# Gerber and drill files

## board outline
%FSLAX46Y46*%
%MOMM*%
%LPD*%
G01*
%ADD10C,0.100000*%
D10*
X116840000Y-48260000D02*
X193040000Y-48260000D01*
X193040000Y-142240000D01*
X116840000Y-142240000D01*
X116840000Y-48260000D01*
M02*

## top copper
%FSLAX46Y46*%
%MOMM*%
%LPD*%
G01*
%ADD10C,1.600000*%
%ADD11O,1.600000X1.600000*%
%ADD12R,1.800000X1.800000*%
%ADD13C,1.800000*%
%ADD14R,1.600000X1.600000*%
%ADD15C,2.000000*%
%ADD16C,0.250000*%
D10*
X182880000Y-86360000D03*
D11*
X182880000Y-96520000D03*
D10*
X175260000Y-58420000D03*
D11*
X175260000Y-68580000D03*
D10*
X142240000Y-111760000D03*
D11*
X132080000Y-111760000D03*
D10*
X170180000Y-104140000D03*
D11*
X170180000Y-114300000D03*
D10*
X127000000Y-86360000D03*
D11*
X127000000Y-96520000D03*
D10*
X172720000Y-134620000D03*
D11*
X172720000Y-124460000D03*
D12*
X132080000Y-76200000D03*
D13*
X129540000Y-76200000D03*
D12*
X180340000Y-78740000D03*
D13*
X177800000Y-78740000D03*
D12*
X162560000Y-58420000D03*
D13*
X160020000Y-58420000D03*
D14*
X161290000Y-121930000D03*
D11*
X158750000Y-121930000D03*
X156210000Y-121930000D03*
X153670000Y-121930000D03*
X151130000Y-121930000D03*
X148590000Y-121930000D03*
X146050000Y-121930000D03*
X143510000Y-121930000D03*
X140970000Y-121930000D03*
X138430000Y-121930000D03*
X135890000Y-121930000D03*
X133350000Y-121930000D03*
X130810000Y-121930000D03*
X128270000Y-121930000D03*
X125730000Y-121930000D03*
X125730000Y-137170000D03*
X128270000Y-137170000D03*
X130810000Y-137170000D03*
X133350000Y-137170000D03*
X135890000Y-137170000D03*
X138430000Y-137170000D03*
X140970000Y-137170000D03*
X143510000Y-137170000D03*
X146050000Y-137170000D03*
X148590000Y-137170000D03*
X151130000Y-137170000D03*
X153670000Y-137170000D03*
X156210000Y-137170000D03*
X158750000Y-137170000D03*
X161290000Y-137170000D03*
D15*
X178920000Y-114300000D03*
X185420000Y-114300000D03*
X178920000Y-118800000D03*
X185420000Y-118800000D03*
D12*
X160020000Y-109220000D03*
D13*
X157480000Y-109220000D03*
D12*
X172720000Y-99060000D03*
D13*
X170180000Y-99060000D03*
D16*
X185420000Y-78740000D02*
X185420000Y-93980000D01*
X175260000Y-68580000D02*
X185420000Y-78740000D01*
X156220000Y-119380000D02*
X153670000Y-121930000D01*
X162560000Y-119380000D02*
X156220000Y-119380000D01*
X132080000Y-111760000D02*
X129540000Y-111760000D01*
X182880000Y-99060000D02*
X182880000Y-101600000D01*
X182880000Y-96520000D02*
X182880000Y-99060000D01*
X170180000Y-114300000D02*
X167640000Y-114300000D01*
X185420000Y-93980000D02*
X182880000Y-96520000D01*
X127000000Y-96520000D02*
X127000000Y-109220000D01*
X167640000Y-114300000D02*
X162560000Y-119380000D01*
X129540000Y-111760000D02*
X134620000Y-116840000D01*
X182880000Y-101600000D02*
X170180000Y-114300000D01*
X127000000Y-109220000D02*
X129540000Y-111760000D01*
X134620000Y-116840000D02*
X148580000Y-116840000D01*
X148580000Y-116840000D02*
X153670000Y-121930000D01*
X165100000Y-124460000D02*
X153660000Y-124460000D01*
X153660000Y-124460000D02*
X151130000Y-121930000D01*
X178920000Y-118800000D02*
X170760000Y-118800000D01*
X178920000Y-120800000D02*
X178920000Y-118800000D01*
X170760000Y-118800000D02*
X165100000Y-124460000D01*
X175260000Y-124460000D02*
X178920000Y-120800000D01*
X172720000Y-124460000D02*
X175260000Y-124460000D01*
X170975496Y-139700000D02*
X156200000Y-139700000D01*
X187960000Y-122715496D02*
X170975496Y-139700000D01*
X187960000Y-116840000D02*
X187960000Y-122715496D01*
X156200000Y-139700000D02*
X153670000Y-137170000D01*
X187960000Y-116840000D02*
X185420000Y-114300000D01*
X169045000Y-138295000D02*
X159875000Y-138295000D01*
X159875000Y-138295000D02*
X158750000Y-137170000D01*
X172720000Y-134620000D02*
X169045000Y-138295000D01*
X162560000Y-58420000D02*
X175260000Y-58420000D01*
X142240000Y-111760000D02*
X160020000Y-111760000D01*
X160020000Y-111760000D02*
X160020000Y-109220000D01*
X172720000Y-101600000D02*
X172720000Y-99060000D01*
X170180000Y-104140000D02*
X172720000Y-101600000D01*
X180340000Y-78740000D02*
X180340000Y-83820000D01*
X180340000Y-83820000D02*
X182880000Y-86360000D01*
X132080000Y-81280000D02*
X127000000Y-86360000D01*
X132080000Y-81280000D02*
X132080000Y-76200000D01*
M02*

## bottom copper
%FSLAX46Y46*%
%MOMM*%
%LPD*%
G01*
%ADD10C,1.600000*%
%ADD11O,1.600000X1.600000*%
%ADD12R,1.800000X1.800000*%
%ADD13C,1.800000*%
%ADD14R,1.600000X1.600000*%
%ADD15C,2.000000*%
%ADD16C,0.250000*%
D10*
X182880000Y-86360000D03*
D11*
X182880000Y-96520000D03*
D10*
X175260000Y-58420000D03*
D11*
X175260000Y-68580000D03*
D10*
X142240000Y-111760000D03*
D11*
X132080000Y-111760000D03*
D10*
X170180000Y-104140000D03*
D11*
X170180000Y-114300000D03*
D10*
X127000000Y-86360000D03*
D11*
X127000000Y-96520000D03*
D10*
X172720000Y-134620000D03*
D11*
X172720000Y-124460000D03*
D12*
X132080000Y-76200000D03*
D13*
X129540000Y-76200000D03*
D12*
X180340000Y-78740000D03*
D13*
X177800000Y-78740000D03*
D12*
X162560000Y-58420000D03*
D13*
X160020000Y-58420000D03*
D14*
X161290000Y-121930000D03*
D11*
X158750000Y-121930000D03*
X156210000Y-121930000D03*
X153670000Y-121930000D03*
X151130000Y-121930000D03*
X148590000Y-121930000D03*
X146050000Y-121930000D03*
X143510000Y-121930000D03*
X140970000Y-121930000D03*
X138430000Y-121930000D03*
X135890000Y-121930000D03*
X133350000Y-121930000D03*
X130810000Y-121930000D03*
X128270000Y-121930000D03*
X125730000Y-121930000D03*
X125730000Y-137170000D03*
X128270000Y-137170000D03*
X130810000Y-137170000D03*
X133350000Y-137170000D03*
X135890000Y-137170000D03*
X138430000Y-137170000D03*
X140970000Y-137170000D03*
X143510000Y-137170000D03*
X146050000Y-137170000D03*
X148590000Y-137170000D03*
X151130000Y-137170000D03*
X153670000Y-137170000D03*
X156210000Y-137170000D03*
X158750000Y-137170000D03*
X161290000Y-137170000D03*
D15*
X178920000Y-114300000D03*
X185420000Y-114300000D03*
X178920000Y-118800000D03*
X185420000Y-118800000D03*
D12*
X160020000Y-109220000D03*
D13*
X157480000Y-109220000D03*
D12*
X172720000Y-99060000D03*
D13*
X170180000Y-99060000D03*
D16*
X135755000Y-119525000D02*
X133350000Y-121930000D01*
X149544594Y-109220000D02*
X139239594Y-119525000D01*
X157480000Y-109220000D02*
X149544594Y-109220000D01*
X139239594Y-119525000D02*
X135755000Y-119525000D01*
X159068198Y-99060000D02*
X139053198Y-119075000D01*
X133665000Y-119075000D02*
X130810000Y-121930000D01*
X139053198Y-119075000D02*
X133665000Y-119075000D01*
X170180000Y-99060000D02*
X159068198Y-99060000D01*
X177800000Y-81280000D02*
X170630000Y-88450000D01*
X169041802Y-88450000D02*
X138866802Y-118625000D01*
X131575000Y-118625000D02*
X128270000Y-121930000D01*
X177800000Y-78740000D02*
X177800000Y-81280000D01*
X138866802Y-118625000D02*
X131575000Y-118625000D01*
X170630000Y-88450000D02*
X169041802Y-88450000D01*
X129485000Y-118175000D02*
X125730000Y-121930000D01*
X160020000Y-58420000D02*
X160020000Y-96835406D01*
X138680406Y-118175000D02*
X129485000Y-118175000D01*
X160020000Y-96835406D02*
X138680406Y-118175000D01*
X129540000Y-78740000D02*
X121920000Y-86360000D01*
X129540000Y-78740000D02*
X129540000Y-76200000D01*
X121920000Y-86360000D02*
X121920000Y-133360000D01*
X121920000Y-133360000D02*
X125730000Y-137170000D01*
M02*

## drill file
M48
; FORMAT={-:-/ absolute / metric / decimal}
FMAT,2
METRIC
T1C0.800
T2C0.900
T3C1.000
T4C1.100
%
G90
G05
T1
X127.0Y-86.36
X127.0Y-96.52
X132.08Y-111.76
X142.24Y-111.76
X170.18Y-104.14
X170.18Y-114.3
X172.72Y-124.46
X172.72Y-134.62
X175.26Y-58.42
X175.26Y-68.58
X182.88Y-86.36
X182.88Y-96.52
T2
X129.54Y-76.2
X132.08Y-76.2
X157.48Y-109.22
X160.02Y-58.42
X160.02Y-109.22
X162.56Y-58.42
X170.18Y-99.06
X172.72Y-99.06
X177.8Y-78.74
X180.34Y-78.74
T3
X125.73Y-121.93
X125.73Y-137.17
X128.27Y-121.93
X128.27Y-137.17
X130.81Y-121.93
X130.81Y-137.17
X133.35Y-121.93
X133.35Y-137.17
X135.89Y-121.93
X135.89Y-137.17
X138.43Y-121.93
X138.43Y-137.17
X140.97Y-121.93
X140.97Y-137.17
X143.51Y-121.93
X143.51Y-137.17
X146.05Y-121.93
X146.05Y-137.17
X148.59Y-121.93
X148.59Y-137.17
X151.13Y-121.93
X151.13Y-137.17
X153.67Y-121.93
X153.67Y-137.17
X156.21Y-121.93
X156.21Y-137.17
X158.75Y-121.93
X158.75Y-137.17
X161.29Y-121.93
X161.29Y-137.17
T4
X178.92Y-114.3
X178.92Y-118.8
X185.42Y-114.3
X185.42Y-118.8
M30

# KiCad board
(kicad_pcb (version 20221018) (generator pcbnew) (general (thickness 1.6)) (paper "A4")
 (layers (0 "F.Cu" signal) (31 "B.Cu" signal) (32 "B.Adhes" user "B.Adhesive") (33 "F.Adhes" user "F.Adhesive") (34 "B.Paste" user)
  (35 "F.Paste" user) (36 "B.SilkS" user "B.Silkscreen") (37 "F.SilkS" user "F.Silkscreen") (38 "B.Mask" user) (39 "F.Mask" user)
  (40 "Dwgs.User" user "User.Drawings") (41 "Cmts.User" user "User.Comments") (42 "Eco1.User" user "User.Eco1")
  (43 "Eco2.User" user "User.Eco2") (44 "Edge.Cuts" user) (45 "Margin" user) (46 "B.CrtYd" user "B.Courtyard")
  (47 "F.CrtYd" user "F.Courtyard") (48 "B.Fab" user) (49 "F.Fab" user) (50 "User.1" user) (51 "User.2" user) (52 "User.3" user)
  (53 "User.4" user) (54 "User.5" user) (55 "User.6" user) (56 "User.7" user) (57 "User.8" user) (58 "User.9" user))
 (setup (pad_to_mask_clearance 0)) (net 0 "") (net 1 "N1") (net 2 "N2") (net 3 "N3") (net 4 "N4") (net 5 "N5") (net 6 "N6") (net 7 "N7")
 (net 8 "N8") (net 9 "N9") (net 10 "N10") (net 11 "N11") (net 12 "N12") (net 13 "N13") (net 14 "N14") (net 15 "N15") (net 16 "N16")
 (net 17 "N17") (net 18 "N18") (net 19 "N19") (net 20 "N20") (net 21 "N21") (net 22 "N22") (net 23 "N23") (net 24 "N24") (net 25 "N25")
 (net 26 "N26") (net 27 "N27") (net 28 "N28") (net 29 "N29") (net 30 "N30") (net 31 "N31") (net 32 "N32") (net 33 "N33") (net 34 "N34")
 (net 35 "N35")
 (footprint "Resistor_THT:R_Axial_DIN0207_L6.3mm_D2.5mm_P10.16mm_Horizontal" (layer "F.Cu") (at 182.88 86.36 -90)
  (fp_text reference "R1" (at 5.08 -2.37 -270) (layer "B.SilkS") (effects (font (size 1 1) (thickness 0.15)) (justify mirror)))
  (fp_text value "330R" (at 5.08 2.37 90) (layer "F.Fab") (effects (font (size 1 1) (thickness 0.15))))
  (pad "1" thru_hole circle (at 0 0 270) (size 1.6 1.6) (drill 0.8) (layers "*.Cu" "*.Mask") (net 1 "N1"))
  (pad "2" thru_hole oval (at 10.16 0 270) (size 1.6 1.6) (drill 0.8) (layers "*.Cu" "*.Mask") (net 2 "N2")))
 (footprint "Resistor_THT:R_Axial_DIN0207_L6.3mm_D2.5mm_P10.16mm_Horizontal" (layer "F.Cu") (at 175.26 58.42 -90)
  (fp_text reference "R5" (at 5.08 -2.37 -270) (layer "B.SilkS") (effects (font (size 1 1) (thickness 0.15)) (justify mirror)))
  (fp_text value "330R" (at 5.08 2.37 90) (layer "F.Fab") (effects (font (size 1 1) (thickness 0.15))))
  (pad "1" thru_hole circle (at 0 0 270) (size 1.6 1.6) (drill 0.8) (layers "*.Cu" "*.Mask") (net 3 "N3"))
  (pad "2" thru_hole oval (at 10.16 0 270) (size 1.6 1.6) (drill 0.8) (layers "*.Cu" "*.Mask") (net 2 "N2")))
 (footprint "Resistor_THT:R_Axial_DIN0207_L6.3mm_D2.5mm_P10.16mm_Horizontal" (layer "F.Cu") (at 142.24 111.76 180)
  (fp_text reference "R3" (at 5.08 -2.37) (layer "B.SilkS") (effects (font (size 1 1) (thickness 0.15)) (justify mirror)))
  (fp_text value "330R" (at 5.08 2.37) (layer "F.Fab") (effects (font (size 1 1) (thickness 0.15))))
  (pad "1" thru_hole circle (at 0 0 180) (size 1.6 1.6) (drill 0.8) (layers "*.Cu" "*.Mask") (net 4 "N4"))
  (pad "2" thru_hole oval (at 10.16 0 180) (size 1.6 1.6) (drill 0.8) (layers "*.Cu" "*.Mask") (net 2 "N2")))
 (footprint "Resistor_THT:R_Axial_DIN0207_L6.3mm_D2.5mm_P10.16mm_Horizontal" (layer "F.Cu") (at 170.18 104.14 -90)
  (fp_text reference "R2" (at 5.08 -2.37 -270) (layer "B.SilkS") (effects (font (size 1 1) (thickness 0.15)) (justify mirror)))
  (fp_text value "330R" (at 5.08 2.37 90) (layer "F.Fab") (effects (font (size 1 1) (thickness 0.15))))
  (pad "1" thru_hole circle (at 0 0 270) (size 1.6 1.6) (drill 0.8) (layers "*.Cu" "*.Mask") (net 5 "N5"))
  (pad "2" thru_hole oval (at 10.16 0 270) (size 1.6 1.6) (drill 0.8) (layers "*.Cu" "*.Mask") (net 2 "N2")))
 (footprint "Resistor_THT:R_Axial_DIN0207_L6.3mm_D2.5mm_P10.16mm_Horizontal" (layer "F.Cu") (at 127 86.36 -90)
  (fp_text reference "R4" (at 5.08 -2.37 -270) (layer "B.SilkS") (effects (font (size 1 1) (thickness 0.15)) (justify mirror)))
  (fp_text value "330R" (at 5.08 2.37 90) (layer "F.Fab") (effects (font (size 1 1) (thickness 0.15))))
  (pad "1" thru_hole circle (at 0 0 270) (size 1.6 1.6) (drill 0.8) (layers "*.Cu" "*.Mask") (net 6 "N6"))
  (pad "2" thru_hole oval (at 10.16 0 270) (size 1.6 1.6) (drill 0.8) (layers "*.Cu" "*.Mask") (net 2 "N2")))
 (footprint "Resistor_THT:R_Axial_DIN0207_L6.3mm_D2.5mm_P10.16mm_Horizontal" (layer "F.Cu") (at 172.72 134.62 90)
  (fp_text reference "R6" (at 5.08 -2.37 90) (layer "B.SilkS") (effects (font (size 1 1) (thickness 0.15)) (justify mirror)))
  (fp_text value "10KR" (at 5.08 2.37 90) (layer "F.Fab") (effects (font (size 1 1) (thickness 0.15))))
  (pad "1" thru_hole circle (at 0 0 90) (size 1.6 1.6) (drill 0.8) (layers "*.Cu" "*.Mask") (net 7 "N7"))
  (pad "2" thru_hole oval (at 10.16 0 90) (size 1.6 1.6) (drill 0.8) (layers "*.Cu" "*.Mask") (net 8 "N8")))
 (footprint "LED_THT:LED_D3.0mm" (layer "F.Cu") (at 132.08 76.2 180)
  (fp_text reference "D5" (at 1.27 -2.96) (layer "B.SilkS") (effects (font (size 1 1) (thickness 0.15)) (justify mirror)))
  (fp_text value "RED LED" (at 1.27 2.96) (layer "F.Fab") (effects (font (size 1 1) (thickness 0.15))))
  (pad "1" thru_hole rect (at 0 0 180) (size 1.8 1.8) (drill 0.9) (layers "*.Cu" "*.Mask") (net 6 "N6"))
  (pad "2" thru_hole circle (at 2.54 0 180) (size 1.8 1.8) (drill 0.9) (layers "*.Cu" "*.Mask") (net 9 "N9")))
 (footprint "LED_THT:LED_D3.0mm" (layer "F.Cu") (at 180.34 78.74 180)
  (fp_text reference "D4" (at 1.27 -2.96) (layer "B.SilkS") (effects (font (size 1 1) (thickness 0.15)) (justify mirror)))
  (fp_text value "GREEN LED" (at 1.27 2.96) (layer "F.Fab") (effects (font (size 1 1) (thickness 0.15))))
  (pad "1" thru_hole rect (at 0 0 180) (size 1.8 1.8) (drill 0.9) (layers "*.Cu" "*.Mask") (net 1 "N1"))
  (pad "2" thru_hole circle (at 2.54 0 180) (size 1.8 1.8) (drill 0.9) (layers "*.Cu" "*.Mask") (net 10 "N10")))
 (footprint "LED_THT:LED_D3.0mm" (layer "F.Cu") (at 162.56 58.42 180)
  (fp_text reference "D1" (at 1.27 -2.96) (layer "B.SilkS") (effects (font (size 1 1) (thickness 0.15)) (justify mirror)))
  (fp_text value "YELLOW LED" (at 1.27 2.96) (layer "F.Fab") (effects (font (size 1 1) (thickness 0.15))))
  (pad "1" thru_hole rect (at 0 0 180) (size 1.8 1.8) (drill 0.9) (layers "*.Cu" "*.Mask") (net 3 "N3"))
  (pad "2" thru_hole circle (at 2.54 0 180) (size 1.8 1.8) (drill 0.9) (layers "*.Cu" "*.Mask") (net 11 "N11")))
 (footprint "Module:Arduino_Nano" (layer "F.Cu") (at 161.29 121.93 -90)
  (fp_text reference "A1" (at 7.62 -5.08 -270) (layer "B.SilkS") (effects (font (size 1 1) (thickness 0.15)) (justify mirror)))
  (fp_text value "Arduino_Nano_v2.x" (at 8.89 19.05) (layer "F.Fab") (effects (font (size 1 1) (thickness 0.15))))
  (pad "1" thru_hole rect (at 0 0 270) (size 1.6 1.6) (drill 1) (layers "*.Cu" "*.Mask") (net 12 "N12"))
  (pad "2" thru_hole oval (at 0 2.54 270) (size 1.6 1.6) (drill 1) (layers "*.Cu" "*.Mask") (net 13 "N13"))
  (pad "3" thru_hole oval (at 0 5.08 270) (size 1.6 1.6) (drill 1) (layers "*.Cu" "*.Mask") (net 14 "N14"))
  (pad "4" thru_hole oval (at 0 7.62 270) (size 1.6 1.6) (drill 1) (layers "*.Cu" "*.Mask") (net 2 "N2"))
  (pad "5" thru_hole oval (at 0 10.16 270) (size 1.6 1.6) (drill 1) (layers "*.Cu" "*.Mask") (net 8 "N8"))
  (pad "6" thru_hole oval (at 0 12.7 270) (size 1.6 1.6) (drill 1) (layers "*.Cu" "*.Mask") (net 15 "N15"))
  (pad "7" thru_hole oval (at 0 15.24 270) (size 1.6 1.6) (drill 1) (layers "*.Cu" "*.Mask") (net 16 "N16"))
  (pad "8" thru_hole oval (at 0 17.78 270) (size 1.6 1.6) (drill 1) (layers "*.Cu" "*.Mask") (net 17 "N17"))
  (pad "9" thru_hole oval (at 0 20.32 270) (size 1.6 1.6) (drill 1) (layers "*.Cu" "*.Mask") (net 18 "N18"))
  (pad "10" thru_hole oval (at 0 22.86 270) (size 1.6 1.6) (drill 1) (layers "*.Cu" "*.Mask") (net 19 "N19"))
  (pad "11" thru_hole oval (at 0 25.4 270) (size 1.6 1.6) (drill 1) (layers "*.Cu" "*.Mask") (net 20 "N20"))
  (pad "12" thru_hole oval (at 0 27.94 270) (size 1.6 1.6) (drill 1) (layers "*.Cu" "*.Mask") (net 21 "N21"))
  (pad "13" thru_hole oval (at 0 30.48 270) (size 1.6 1.6) (drill 1) (layers "*.Cu" "*.Mask") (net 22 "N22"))
  (pad "14" thru_hole oval (at 0 33.02 270) (size 1.6 1.6) (drill 1) (layers "*.Cu" "*.Mask") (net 10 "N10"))
  (pad "15" thru_hole oval (at 0 35.56 270) (size 1.6 1.6) (drill 1) (layers "*.Cu" "*.Mask") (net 11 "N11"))
  (pad "16" thru_hole oval (at 15.24 35.56 270) (size 1.6 1.6) (drill 1) (layers "*.Cu" "*.Mask") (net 9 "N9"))
  (pad "17" thru_hole oval (at 15.24 33.02 270) (size 1.6 1.6) (drill 1) (layers "*.Cu" "*.Mask") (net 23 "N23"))
  (pad "18" thru_hole oval (at 15.24 30.48 270) (size 1.6 1.6) (drill 1) (layers "*.Cu" "*.Mask") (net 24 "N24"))
  (pad "19" thru_hole oval (at 15.24 27.94 270) (size 1.6 1.6) (drill 1) (layers "*.Cu" "*.Mask") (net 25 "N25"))
  (pad "20" thru_hole oval (at 15.24 25.4 270) (size 1.6 1.6) (drill 1) (layers "*.Cu" "*.Mask") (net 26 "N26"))
  (pad "21" thru_hole oval (at 15.24 22.86 270) (size 1.6 1.6) (drill 1) (layers "*.Cu" "*.Mask") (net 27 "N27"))
  (pad "22" thru_hole oval (at 15.24 20.32 270) (size 1.6 1.6) (drill 1) (layers "*.Cu" "*.Mask") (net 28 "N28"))
  (pad "23" thru_hole oval (at 15.24 17.78 270) (size 1.6 1.6) (drill 1) (layers "*.Cu" "*.Mask") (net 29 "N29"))
  (pad "24" thru_hole oval (at 15.24 15.24 270) (size 1.6 1.6) (drill 1) (layers "*.Cu" "*.Mask") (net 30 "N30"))
  (pad "25" thru_hole oval (at 15.24 12.7 270) (size 1.6 1.6) (drill 1) (layers "*.Cu" "*.Mask") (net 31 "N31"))
  (pad "26" thru_hole oval (at 15.24 10.16 270) (size 1.6 1.6) (drill 1) (layers "*.Cu" "*.Mask") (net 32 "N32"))
  (pad "27" thru_hole oval (at 15.24 7.62 270) (size 1.6 1.6) (drill 1) (layers "*.Cu" "*.Mask") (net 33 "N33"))
  (pad "28" thru_hole oval (at 15.24 5.08 270) (size 1.6 1.6) (drill 1) (layers "*.Cu" "*.Mask") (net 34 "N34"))
  (pad "29" thru_hole oval (at 15.24 2.54 270) (size 1.6 1.6) (drill 1) (layers "*.Cu" "*.Mask") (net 7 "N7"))
  (pad "30" thru_hole oval (at 15.24 0 270) (size 1.6 1.6) (drill 1) (layers "*.Cu" "*.Mask") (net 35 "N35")))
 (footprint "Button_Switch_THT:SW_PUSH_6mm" (layer "F.Cu") (at 178.92 114.3)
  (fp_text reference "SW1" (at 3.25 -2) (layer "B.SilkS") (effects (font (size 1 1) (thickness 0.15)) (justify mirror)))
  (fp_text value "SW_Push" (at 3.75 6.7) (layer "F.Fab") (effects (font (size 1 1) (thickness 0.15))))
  (pad "1" thru_hole circle (at 0 0 90) (size 2 2) (drill 1.1) (layers "*.Cu" "*.Mask") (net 33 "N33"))
  (pad "1" thru_hole circle (at 6.5 0 90) (size 2 2) (drill 1.1) (layers "*.Cu" "*.Mask") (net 33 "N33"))
  (pad "2" thru_hole circle (at 0 4.5 90) (size 2 2) (drill 1.1) (layers "*.Cu" "*.Mask") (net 8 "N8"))
  (pad "2" thru_hole circle (at 6.5 4.5 90) (size 2 2) (drill 1.1) (layers "*.Cu" "*.Mask") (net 8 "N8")))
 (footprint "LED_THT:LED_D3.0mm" (layer "F.Cu") (at 160.02 109.22 180)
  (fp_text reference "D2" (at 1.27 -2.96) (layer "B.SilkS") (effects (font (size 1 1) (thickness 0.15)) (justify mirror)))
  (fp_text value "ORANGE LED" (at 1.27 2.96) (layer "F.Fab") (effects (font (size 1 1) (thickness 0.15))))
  (pad "1" thru_hole rect (at 0 0 180) (size 1.8 1.8) (drill 0.9) (layers "*.Cu" "*.Mask") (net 4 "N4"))
  (pad "2" thru_hole circle (at 2.54 0 180) (size 1.8 1.8) (drill 0.9) (layers "*.Cu" "*.Mask") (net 21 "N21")))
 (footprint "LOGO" (layer "F.Cu") (at 154.94 83.82)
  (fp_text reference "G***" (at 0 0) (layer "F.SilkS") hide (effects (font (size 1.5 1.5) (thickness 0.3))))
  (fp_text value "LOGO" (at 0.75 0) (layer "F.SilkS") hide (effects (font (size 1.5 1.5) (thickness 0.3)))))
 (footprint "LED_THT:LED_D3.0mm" (layer "F.Cu") (at 172.72 99.06 180)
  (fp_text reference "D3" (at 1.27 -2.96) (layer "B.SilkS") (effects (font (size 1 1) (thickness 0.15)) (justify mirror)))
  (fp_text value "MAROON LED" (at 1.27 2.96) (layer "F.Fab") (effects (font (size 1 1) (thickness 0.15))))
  (pad "1" thru_hole rect (at 0 0 180) (size 1.8 1.8) (drill 0.9) (layers "*.Cu" "*.Mask") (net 5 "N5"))
  (pad "2" thru_hole circle (at 2.54 0 180) (size 1.8 1.8) (drill 0.9) (layers "*.Cu" "*.Mask") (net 22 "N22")))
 (gr_rect (start 116.84 48.26) (end 193.04 142.24) (stroke (width 0.1) (type default)) (fill none) (layer "Edge.Cuts"))
 (segment (start 185.42 78.74) (end 185.42 93.98) (width 0.25) (layer "F.Cu") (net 2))
 (segment (start 175.26 68.58) (end 185.42 78.74) (width 0.25) (layer "F.Cu") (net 2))
 (segment (start 156.22 119.38) (end 153.67 121.93) (width 0.25) (layer "F.Cu") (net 2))
 (segment (start 162.56 119.38) (end 156.22 119.38) (width 0.25) (layer "F.Cu") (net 2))
 (segment (start 132.08 111.76) (end 129.54 111.76) (width 0.25) (layer "F.Cu") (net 2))
 (segment (start 182.88 99.06) (end 182.88 101.6) (width 0.25) (layer "F.Cu") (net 2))
 (segment (start 182.88 96.52) (end 182.88 99.06) (width 0.25) (layer "F.Cu") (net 2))
 (segment (start 170.18 114.3) (end 167.64 114.3) (width 0.25) (layer "F.Cu") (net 2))
 (segment (start 185.42 93.98) (end 182.88 96.52) (width 0.25) (layer "F.Cu") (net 2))
 (segment (start 127 96.52) (end 127 109.22) (width 0.25) (layer "F.Cu") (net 2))
 (segment (start 167.64 114.3) (end 162.56 119.38) (width 0.25) (layer "F.Cu") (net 2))
 (segment (start 129.54 111.76) (end 134.62 116.84) (width 0.25) (layer "F.Cu") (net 2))
 (segment (start 182.88 101.6) (end 170.18 114.3) (width 0.25) (layer "F.Cu") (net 2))
 (segment (start 127 109.22) (end 129.54 111.76) (width 0.25) (layer "F.Cu") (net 2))
 (segment (start 134.62 116.84) (end 148.58 116.84) (width 0.25) (layer "F.Cu") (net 2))
 (segment (start 148.58 116.84) (end 153.67 121.93) (width 0.25) (layer "F.Cu") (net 2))
 (segment (start 165.1 124.46) (end 153.66 124.46) (width 0.25) (layer "F.Cu") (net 8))
 (segment (start 153.66 124.46) (end 151.13 121.93) (width 0.25) (layer "F.Cu") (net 8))
 (segment (start 178.92 118.8) (end 170.76 118.8) (width 0.25) (layer "F.Cu") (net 8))
 (segment (start 178.92 120.8) (end 178.92 118.8) (width 0.25) (layer "F.Cu") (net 8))
 (segment (start 170.76 118.8) (end 165.1 124.46) (width 0.25) (layer "F.Cu") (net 8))
 (segment (start 175.26 124.46) (end 178.92 120.8) (width 0.25) (layer "F.Cu") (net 8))
 (segment (start 172.72 124.46) (end 175.26 124.46) (width 0.25) (layer "F.Cu") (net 8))
 (segment (start 135.755 119.525) (end 133.35 121.93) (width 0.25) (layer "B.Cu") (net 21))
 (segment (start 149.544594 109.22) (end 139.239594 119.525) (width 0.25) (layer "B.Cu") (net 21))
 (segment (start 157.48 109.22) (end 149.544594 109.22) (width 0.25) (layer "B.Cu") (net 21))
 (segment (start 139.239594 119.525) (end 135.755 119.525) (width 0.25) (layer "B.Cu") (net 21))
 (segment (start 159.068198 99.06) (end 139.053198 119.075) (width 0.25) (layer "B.Cu") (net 22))
 (segment (start 133.665 119.075) (end 130.81 121.93) (width 0.25) (layer "B.Cu") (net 22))
 (segment (start 139.053198 119.075) (end 133.665 119.075) (width 0.25) (layer "B.Cu") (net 22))
 (segment (start 170.18 99.06) (end 159.068198 99.06) (width 0.25) (layer "B.Cu") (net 22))
 (segment (start 177.8 81.28) (end 170.63 88.45) (width 0.25) (layer "B.Cu") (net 10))
 (segment (start 169.041802 88.45) (end 138.866802 118.625) (width 0.25) (layer "B.Cu") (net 10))
 (segment (start 131.575 118.625) (end 128.27 121.93) (width 0.25) (layer "B.Cu") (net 10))
 (segment (start 177.8 78.74) (end 177.8 81.28) (width 0.25) (layer "B.Cu") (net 10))
 (segment (start 138.866802 118.625) (end 131.575 118.625) (width 0.25) (layer "B.Cu") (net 10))
 (segment (start 170.63 88.45) (end 169.041802 88.45) (width 0.25) (layer "B.Cu") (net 10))
 (segment (start 129.485 118.175) (end 125.73 121.93) (width 0.25) (layer "B.Cu") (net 11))
 (segment (start 160.02 58.42) (end 160.02 96.835406) (width 0.25) (layer "B.Cu") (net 11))
 (segment (start 138.680406 118.175) (end 129.485 118.175) (width 0.25) (layer "B.Cu") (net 11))
 (segment (start 160.02 96.835406) (end 138.680406 118.175) (width 0.25) (layer "B.Cu") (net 11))
 (segment (start 129.54 78.74) (end 121.92 86.36) (width 0.25) (layer "B.Cu") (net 9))
 (segment (start 129.54 78.74) (end 129.54 76.2) (width 0.25) (layer "B.Cu") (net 9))
 (segment (start 121.92 86.36) (end 121.92 133.36) (width 0.25) (layer "B.Cu") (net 9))
 (segment (start 121.92 133.36) (end 125.73 137.17) (width 0.25) (layer "B.Cu") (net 9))
 (segment (start 170.975496 139.7) (end 156.2 139.7) (width 0.25) (layer "F.Cu") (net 33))
 (segment (start 187.96 122.715496) (end 170.975496 139.7) (width 0.25) (layer "F.Cu") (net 33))
 (segment (start 187.96 116.84) (end 187.96 122.715496) (width 0.25) (layer "F.Cu") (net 33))
 (segment (start 156.2 139.7) (end 153.67 137.17) (width 0.25) (layer "F.Cu") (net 33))
 (segment (start 187.96 116.84) (end 185.42 114.3) (width 0.25) (layer "F.Cu") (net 33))
 (segment (start 169.045 138.295) (end 159.875 138.295) (width 0.25) (layer "F.Cu") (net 7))
 (segment (start 159.875 138.295) (end 158.75 137.17) (width 0.25) (layer "F.Cu") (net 7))
 (segment (start 172.72 134.62) (end 169.045 138.295) (width 0.25) (layer "F.Cu") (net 7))
 (segment (start 162.56 58.42) (end 175.26 58.42) (width 0.25) (layer "F.Cu") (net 3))
 (segment (start 142.24 111.76) (end 160.02 111.76) (width 0.25) (layer "F.Cu") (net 4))
 (segment (start 160.02 111.76) (end 160.02 109.22) (width 0.25) (layer "F.Cu") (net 4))
 (segment (start 172.72 101.6) (end 172.72 99.06) (width 0.25) (layer "F.Cu") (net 5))
 (segment (start 170.18 104.14) (end 172.72 101.6) (width 0.25) (layer "F.Cu") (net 5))
 (segment (start 180.34 78.74) (end 180.34 83.82) (width 0.25) (layer "F.Cu") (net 1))
 (segment (start 180.34 83.82) (end 182.88 86.36) (width 0.25) (layer "F.Cu") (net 1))
 (segment (start 132.08 81.28) (end 127 86.36) (width 0.25) (layer "F.Cu") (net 6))
 (segment (start 132.08 81.28) (end 132.08 76.2) (width 0.25) (layer "F.Cu") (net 6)))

